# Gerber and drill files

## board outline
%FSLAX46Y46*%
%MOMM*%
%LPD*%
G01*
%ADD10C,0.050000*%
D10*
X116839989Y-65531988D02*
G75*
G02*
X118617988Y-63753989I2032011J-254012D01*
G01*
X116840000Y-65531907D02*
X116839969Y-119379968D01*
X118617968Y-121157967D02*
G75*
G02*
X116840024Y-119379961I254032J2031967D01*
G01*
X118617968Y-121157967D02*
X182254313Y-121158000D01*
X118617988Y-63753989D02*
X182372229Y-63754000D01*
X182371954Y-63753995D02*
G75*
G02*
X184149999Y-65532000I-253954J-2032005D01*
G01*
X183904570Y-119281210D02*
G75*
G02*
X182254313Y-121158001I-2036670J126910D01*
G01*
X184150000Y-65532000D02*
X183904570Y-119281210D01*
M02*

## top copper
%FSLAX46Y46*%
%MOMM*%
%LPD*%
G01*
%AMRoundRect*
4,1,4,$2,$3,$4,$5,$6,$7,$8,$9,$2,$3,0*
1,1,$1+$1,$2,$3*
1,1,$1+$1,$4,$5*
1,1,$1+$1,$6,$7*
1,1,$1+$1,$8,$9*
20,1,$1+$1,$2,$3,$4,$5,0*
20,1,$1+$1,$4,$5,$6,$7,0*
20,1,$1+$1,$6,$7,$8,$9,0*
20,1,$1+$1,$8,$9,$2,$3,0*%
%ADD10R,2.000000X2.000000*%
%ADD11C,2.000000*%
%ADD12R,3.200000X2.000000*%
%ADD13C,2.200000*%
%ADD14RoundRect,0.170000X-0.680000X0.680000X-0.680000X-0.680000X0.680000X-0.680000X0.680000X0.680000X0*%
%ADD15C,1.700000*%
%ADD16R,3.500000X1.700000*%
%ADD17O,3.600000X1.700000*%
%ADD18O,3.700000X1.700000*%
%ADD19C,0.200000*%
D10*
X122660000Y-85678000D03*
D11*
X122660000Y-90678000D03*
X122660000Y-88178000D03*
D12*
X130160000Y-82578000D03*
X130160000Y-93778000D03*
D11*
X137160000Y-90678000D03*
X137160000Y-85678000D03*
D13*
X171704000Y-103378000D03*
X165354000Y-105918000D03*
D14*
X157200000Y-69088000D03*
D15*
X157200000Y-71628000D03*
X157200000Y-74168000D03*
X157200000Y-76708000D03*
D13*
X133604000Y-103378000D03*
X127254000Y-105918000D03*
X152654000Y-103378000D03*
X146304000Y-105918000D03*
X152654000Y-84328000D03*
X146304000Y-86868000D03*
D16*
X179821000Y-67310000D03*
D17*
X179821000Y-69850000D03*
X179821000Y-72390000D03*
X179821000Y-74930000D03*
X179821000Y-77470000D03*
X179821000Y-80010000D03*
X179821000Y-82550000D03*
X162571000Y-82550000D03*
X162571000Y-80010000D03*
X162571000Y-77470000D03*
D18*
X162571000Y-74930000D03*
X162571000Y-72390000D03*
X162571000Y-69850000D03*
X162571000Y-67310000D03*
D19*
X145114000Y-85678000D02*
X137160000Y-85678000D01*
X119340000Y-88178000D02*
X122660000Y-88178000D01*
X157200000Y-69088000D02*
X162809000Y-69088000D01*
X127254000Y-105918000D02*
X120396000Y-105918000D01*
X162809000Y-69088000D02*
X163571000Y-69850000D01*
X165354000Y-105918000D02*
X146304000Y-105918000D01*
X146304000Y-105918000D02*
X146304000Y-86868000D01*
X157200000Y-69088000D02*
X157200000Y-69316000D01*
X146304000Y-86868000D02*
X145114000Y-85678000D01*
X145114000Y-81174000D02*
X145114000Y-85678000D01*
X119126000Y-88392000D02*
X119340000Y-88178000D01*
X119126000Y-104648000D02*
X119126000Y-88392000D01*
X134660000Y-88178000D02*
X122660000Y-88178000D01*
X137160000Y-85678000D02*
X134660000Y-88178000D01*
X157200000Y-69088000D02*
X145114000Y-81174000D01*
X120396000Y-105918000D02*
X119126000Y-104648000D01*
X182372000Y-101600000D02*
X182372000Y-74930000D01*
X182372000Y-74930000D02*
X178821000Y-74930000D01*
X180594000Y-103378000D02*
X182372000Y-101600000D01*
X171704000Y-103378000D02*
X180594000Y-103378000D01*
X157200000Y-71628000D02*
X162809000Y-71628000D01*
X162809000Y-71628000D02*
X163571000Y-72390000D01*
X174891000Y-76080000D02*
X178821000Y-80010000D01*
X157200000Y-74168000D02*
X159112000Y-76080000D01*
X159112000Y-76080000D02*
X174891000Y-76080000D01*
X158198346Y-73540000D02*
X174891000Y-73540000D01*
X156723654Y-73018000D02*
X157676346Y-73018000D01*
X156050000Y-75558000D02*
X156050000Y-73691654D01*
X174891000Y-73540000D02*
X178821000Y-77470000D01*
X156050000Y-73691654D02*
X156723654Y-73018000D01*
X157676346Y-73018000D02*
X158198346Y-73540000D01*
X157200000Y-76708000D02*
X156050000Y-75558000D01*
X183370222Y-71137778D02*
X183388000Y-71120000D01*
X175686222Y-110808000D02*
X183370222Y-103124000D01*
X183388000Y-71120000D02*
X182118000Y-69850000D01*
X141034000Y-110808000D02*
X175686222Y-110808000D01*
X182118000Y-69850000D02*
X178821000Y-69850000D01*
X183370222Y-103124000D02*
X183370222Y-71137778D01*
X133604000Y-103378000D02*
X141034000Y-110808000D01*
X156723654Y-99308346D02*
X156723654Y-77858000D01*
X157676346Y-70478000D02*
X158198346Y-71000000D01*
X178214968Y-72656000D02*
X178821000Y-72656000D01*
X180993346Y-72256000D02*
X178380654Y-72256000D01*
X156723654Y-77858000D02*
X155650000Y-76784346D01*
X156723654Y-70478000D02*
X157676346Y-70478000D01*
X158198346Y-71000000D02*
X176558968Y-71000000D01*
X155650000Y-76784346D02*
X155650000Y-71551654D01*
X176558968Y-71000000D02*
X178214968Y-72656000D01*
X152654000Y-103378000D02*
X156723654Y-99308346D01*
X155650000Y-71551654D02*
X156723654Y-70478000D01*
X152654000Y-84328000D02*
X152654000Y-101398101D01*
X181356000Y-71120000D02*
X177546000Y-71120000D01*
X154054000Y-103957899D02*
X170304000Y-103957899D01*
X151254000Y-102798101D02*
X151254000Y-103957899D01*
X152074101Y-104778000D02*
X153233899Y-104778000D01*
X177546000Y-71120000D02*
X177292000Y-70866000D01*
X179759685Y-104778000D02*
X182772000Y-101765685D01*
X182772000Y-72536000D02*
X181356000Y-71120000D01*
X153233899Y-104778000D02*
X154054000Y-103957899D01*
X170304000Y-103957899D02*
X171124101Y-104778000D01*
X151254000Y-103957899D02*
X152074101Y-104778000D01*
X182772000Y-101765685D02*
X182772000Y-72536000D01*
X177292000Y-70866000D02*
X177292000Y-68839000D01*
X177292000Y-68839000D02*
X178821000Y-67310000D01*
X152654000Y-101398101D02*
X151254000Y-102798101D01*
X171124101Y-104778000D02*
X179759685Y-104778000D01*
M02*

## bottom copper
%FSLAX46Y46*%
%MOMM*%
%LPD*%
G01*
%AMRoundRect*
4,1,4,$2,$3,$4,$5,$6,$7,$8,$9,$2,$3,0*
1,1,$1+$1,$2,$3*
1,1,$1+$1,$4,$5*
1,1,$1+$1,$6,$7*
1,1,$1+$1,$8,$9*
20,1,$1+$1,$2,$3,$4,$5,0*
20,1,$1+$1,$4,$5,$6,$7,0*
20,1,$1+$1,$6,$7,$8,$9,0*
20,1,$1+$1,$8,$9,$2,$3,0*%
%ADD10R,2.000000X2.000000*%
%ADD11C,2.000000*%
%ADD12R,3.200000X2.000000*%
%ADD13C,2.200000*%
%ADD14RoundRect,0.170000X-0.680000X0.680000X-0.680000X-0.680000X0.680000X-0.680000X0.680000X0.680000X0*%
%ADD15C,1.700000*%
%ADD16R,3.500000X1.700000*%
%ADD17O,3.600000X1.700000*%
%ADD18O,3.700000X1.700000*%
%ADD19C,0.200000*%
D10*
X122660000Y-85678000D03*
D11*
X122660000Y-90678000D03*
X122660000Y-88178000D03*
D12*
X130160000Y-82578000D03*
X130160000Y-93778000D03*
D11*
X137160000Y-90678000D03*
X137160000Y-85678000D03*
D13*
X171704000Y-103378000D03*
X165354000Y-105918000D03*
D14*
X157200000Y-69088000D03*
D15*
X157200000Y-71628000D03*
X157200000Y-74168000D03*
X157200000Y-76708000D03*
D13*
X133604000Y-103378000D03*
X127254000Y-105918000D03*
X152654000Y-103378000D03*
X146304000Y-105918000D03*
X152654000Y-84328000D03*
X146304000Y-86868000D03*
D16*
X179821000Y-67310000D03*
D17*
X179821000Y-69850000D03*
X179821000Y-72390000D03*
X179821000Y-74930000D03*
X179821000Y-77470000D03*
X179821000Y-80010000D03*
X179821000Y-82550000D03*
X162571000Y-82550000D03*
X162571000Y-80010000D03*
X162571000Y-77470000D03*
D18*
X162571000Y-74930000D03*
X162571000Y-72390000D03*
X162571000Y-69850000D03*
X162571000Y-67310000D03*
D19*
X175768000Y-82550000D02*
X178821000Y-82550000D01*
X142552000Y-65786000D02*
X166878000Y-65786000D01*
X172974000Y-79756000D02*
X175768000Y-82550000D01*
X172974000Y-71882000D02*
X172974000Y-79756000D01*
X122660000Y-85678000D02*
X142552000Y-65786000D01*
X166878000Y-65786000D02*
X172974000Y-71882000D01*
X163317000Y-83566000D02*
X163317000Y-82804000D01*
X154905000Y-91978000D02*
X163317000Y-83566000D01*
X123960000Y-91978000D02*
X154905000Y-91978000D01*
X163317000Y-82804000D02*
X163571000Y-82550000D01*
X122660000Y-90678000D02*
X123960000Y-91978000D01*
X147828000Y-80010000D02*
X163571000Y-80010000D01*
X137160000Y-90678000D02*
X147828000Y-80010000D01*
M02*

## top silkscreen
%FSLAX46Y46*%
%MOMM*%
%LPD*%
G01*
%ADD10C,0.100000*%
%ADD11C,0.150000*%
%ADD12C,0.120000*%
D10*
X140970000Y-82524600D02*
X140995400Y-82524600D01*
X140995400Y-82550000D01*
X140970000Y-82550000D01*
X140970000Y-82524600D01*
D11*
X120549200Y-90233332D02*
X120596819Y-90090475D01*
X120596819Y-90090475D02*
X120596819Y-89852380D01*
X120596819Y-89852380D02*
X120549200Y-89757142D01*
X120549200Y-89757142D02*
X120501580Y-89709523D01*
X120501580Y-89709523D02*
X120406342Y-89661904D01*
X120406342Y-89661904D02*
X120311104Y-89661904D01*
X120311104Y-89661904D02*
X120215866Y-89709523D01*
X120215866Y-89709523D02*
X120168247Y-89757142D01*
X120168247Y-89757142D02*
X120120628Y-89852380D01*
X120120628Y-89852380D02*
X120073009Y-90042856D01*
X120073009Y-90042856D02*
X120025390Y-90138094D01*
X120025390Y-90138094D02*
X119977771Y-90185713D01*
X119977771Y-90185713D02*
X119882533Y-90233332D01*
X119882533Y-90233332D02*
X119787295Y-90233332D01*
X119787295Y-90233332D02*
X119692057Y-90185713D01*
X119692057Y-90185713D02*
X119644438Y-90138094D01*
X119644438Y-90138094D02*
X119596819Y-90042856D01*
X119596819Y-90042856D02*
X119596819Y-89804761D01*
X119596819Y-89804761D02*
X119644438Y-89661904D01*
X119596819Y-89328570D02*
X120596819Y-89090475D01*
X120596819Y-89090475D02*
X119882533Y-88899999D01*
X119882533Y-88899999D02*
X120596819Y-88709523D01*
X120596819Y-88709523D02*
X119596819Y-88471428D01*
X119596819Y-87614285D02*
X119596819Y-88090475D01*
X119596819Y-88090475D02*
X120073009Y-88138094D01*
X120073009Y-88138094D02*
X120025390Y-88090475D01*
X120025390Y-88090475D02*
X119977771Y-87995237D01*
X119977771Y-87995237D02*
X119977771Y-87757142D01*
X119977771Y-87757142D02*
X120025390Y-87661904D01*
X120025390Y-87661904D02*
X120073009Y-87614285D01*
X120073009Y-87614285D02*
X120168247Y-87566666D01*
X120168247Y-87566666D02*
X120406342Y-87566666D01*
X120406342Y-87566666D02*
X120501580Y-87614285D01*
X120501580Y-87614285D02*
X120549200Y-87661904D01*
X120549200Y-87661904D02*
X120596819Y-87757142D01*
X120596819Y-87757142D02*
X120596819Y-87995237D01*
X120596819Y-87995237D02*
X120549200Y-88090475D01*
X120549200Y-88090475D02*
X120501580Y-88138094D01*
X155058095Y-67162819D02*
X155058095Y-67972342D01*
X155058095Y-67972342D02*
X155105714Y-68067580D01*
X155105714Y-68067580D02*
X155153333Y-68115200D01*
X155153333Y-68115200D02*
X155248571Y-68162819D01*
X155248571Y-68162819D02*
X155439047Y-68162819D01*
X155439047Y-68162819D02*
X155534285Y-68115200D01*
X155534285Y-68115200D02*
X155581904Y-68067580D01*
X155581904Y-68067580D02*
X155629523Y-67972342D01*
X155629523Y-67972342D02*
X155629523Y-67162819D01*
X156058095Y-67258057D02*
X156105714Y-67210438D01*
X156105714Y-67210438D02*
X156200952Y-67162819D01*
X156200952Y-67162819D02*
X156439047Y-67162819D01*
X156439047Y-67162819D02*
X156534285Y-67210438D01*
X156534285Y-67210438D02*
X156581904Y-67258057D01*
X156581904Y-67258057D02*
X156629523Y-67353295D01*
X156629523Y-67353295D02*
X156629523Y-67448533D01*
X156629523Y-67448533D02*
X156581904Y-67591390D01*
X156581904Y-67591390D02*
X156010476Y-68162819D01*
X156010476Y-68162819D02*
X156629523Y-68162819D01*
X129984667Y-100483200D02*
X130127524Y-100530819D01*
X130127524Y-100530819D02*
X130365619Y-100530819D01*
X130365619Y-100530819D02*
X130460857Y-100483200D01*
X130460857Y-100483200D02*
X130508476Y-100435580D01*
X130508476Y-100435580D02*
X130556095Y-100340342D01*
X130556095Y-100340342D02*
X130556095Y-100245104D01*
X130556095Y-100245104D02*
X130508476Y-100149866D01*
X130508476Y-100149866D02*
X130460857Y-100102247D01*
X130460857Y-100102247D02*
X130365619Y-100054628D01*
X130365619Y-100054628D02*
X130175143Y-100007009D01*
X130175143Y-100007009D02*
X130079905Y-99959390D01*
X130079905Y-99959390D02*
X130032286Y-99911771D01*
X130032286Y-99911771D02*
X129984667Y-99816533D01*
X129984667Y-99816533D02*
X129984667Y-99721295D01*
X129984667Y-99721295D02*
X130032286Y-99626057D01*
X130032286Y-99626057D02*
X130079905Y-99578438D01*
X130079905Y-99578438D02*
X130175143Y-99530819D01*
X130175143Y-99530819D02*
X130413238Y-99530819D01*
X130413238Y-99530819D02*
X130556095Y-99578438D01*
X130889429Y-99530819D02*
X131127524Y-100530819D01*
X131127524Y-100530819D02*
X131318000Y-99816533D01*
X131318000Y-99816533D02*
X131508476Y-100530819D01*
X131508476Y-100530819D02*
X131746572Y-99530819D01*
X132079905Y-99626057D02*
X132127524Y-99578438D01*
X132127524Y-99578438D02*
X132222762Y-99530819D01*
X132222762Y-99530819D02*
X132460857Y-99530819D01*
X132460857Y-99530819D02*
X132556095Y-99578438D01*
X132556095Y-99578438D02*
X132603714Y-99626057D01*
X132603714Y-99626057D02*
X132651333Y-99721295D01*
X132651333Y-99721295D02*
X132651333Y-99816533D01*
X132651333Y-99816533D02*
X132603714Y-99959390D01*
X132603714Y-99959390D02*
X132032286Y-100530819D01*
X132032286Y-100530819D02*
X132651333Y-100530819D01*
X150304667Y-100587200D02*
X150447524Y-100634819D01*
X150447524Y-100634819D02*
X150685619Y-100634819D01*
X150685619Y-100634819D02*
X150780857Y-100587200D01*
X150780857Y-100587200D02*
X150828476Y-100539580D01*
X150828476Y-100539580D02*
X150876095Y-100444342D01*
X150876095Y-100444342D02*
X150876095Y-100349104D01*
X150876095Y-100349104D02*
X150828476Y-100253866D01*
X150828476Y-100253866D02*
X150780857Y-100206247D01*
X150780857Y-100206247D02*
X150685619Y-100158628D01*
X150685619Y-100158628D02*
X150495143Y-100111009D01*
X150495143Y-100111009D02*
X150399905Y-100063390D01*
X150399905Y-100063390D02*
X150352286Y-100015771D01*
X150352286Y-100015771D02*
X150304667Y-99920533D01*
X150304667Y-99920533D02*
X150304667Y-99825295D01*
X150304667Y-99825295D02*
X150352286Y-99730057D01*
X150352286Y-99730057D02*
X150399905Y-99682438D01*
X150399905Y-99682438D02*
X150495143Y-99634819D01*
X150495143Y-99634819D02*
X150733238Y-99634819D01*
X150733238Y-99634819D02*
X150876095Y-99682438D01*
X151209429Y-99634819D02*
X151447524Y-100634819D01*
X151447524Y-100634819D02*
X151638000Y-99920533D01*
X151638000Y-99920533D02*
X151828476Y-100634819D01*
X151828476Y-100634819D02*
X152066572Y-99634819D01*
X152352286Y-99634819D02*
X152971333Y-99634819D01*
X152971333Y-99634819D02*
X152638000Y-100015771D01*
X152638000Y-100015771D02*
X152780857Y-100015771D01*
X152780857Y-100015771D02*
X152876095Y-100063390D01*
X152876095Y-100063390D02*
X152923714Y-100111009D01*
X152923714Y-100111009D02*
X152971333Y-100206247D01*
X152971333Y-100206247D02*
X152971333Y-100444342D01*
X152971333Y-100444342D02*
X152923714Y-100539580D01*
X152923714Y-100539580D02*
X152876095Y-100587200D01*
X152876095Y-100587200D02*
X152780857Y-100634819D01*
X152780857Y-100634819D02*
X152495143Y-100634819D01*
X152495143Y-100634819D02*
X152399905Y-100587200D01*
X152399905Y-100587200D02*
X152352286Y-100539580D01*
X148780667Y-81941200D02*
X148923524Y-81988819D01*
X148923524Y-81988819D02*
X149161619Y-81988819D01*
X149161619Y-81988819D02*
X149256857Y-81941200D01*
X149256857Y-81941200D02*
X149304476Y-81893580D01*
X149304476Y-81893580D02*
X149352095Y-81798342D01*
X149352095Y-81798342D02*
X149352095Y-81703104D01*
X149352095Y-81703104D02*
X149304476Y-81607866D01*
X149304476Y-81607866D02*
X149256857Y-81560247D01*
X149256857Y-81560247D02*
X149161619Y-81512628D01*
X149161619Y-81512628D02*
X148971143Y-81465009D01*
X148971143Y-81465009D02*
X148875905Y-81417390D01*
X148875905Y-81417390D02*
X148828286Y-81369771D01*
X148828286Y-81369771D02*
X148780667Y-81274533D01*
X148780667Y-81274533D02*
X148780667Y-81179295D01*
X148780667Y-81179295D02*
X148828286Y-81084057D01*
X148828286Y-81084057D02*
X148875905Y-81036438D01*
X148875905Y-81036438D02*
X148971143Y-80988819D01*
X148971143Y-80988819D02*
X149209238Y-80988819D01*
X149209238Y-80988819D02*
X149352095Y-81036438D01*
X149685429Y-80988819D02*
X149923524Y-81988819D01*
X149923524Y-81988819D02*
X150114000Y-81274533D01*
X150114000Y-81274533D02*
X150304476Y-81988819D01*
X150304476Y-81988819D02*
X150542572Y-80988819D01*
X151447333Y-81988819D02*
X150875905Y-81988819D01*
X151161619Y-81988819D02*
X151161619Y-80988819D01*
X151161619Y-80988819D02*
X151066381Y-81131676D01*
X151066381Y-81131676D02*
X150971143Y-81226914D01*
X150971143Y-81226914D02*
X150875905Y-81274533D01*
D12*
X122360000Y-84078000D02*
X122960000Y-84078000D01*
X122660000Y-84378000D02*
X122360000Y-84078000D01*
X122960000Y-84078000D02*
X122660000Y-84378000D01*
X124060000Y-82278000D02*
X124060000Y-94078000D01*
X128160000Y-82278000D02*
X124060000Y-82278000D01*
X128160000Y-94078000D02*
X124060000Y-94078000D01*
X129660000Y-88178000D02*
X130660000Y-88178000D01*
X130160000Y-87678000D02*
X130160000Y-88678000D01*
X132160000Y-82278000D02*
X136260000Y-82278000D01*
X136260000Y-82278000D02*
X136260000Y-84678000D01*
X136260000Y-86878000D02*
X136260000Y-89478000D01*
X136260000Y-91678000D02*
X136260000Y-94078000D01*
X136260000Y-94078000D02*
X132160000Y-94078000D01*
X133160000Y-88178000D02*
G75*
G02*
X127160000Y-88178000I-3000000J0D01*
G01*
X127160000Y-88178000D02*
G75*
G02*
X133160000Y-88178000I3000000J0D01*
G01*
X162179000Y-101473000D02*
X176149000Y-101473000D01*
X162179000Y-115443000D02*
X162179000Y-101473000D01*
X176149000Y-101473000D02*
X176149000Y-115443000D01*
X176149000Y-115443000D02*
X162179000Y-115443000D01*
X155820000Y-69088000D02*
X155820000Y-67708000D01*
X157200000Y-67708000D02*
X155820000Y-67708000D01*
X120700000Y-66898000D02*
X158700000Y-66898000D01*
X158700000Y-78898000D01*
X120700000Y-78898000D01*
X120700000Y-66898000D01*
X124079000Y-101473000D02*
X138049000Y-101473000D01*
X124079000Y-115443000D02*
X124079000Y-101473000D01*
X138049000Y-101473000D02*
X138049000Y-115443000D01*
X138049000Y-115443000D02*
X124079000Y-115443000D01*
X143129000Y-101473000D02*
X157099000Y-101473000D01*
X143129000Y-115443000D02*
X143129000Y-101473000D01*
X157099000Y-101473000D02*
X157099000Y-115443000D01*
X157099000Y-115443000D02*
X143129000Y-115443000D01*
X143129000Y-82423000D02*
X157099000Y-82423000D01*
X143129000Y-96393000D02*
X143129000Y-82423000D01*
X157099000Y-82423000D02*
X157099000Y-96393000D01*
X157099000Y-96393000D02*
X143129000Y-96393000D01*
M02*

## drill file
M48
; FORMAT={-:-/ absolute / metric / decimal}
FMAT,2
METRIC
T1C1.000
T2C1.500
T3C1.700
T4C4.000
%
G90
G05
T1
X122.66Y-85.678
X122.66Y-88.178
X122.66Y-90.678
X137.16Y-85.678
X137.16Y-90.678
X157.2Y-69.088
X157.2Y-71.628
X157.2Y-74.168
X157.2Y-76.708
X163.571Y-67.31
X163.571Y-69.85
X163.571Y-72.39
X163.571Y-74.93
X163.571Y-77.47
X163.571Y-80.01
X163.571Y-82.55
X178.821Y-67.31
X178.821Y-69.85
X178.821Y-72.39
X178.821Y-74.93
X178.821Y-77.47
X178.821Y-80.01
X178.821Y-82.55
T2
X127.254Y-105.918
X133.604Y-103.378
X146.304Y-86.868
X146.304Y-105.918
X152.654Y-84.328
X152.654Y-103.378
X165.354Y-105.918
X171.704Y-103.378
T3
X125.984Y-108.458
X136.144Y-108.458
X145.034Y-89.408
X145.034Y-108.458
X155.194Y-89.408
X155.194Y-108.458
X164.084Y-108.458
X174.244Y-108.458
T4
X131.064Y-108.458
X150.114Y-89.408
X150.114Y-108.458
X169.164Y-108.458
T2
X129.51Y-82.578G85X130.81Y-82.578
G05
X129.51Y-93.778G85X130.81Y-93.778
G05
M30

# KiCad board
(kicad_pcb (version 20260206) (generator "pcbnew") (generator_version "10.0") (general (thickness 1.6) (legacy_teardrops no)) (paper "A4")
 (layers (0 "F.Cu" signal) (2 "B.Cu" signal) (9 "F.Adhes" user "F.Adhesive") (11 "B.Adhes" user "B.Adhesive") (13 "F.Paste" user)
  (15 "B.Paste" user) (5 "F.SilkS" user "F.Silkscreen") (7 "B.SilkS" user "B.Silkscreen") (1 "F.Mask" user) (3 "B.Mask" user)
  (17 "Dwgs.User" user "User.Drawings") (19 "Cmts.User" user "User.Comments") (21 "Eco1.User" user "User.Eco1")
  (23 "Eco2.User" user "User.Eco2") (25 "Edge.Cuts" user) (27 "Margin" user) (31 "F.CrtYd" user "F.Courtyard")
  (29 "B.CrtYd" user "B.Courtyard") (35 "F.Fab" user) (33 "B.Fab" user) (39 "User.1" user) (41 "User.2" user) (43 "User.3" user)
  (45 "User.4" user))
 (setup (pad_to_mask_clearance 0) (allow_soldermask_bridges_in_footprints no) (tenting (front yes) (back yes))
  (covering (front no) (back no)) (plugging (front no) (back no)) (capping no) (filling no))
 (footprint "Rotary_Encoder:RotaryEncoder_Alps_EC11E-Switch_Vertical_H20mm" (layer "F.Cu") (at 122.66 85.678)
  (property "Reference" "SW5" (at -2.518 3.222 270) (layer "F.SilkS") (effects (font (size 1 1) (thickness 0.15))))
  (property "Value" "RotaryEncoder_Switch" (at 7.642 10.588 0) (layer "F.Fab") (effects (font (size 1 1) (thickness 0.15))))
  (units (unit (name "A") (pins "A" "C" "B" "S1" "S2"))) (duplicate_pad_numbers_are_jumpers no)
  (fp_line (start -0.3 -1.6) (end 0.3 -1.6) (stroke (width 0.12) (type solid)) (layer "F.SilkS"))
  (fp_line (start 0 -1.3) (end -0.3 -1.6) (stroke (width 0.12) (type solid)) (layer "F.SilkS"))
  (fp_line (start 0.3 -1.6) (end 0 -1.3) (stroke (width 0.12) (type solid)) (layer "F.SilkS"))
  (fp_line (start 1.4 -3.4) (end 1.4 8.4) (stroke (width 0.12) (type solid)) (layer "F.SilkS"))
  (fp_line (start 5.5 -3.4) (end 1.4 -3.4) (stroke (width 0.12) (type solid)) (layer "F.SilkS"))
  (fp_line (start 5.5 8.4) (end 1.4 8.4) (stroke (width 0.12) (type solid)) (layer "F.SilkS"))
  (fp_line (start 7 2.5) (end 8 2.5) (stroke (width 0.12) (type solid)) (layer "F.SilkS"))
  (fp_line (start 7.5 2) (end 7.5 3) (stroke (width 0.12) (type solid)) (layer "F.SilkS"))
  (fp_line (start 9.5 -3.4) (end 13.6 -3.4) (stroke (width 0.12) (type solid)) (layer "F.SilkS"))
  (fp_line (start 13.6 -3.4) (end 13.6 -1) (stroke (width 0.12) (type solid)) (layer "F.SilkS"))
  (fp_line (start 13.6 1.2) (end 13.6 3.8) (stroke (width 0.12) (type solid)) (layer "F.SilkS"))
  (fp_line (start 13.6 6) (end 13.6 8.4) (stroke (width 0.12) (type solid)) (layer "F.SilkS"))
  (fp_line (start 13.6 8.4) (end 9.5 8.4) (stroke (width 0.12) (type solid)) (layer "F.SilkS"))
  (fp_circle (center 7.5 2.5) (end 10.5 2.5) (stroke (width 0.12) (type solid)) (fill no) (layer "F.SilkS"))
  (pad "A" thru_hole rect (at 0 0) (size 2 2) (drill 1) (layers "*.Cu" "*.Mask") (remove_unused_layers no) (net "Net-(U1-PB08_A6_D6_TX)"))
  (pad "B" thru_hole circle (at 0 5) (size 2 2) (drill 1) (layers "*.Cu" "*.Mask") (remove_unused_layers no) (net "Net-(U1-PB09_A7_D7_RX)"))
  (pad "C" thru_hole circle (at 0 2.5) (size 2 2) (drill 1) (layers "*.Cu" "*.Mask") (remove_unused_layers no) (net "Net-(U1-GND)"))
  (pad "MP" thru_hole rect (at 7.5 -3.1) (size 3.2 2) (drill oval 2.8 1.5) (layers "*.Cu" "*.Mask") (remove_unused_layers no))
  (pad "MP" thru_hole rect (at 7.5 8.1) (size 3.2 2) (drill oval 2.8 1.5) (layers "*.Cu" "*.Mask") (remove_unused_layers no))
  (pad "S1" thru_hole circle (at 14.5 5) (size 2 2) (drill 1) (layers "*.Cu" "*.Mask") (remove_unused_layers no)
   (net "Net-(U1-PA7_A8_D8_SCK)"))
  (pad "S2" thru_hole circle (at 14.5 0) (size 2 2) (drill 1) (layers "*.Cu" "*.Mask") (remove_unused_layers no) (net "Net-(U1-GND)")))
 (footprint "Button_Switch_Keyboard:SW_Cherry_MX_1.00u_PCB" (layer "F.Cu") (at 171.704 103.378)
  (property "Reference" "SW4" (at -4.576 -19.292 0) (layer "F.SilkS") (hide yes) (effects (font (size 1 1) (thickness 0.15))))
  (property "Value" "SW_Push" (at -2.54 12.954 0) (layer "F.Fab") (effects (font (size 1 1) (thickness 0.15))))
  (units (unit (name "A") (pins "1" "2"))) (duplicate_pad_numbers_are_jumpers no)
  (fp_line (start -9.525 -1.905) (end 4.445 -1.905) (stroke (width 0.12) (type solid)) (layer "F.SilkS"))
  (fp_line (start -9.525 12.065) (end -9.525 -1.905) (stroke (width 0.12) (type solid)) (layer "F.SilkS"))
  (fp_line (start 4.445 -1.905) (end 4.445 12.065) (stroke (width 0.12) (type solid)) (layer "F.SilkS"))
  (fp_line (start 4.445 12.065) (end -9.525 12.065) (stroke (width 0.12) (type solid)) (layer "F.SilkS"))
  (pad "" np_thru_hole circle (at -7.62 5.08) (size 1.7 1.7) (drill 1.7) (layers "*.Cu" "*.Mask"))
  (pad "" np_thru_hole circle (at -2.54 5.08) (size 4 4) (drill 4) (layers "*.Cu" "*.Mask"))
  (pad "" np_thru_hole circle (at 2.54 5.08) (size 1.7 1.7) (drill 1.7) (layers "*.Cu" "*.Mask"))
  (pad "1" thru_hole circle (at 0 0) (size 2.2 2.2) (drill 1.5) (layers "*.Cu" "*.Mask") (remove_unused_layers no)
   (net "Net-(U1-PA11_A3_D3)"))
  (pad "2" thru_hole circle (at -6.35 2.54) (size 2.2 2.2) (drill 1.5) (layers "*.Cu" "*.Mask") (remove_unused_layers no)
   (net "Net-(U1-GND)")))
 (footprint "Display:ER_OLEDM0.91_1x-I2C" (layer "F.Cu") (at 157.2 69.088 -90)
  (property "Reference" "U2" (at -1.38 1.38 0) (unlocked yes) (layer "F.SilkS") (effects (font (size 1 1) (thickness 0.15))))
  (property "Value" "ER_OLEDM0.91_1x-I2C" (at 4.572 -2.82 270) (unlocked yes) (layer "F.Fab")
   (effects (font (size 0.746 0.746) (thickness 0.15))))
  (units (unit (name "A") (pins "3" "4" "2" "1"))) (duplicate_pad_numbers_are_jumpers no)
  (fp_line (start 0 1.38) (end -1.38 1.38) (stroke (width 0.12) (type solid)) (layer "F.SilkS"))
  (fp_line (start -1.38 0) (end -1.38 1.38) (stroke (width 0.12) (type solid)) (layer "F.SilkS"))
  (fp_rect (start -2.19 -1.5) (end 9.81 36.5) (stroke (width 0.12) (type solid)) (fill no) (layer "F.SilkS"))
  (pad "1" thru_hole roundrect (at 0 0 270) (size 1.7 1.7) (drill 1) (layers "*.Cu" "*.Mask") (remove_unused_layers no)
   (roundrect_rratio 0.1) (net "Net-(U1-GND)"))
  (pad "2" thru_hole circle (at 2.54 0 270) (size 1.7 1.7) (drill 1) (layers "*.Cu" "*.Mask") (remove_unused_layers no) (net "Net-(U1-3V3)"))
  (pad "3" thru_hole circle (at 5.08 0 270) (size 1.7 1.7) (drill 1) (layers "*.Cu" "*.Mask") (remove_unused_layers no)
   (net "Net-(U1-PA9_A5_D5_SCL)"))
  (pad "4" thru_hole circle (at 7.62 0 270) (size 1.7 1.7) (drill 1) (layers "*.Cu" "*.Mask") (remove_unused_layers no)
   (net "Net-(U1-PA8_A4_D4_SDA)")))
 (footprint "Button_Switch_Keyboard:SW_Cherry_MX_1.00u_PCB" (layer "F.Cu") (at 133.604 103.378)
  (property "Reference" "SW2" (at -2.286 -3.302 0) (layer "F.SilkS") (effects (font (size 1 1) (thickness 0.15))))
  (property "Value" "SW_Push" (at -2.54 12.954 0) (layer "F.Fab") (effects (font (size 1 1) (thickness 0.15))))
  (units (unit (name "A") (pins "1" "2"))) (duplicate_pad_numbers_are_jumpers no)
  (fp_line (start -9.525 -1.905) (end 4.445 -1.905) (stroke (width 0.12) (type solid)) (layer "F.SilkS"))
  (fp_line (start -9.525 12.065) (end -9.525 -1.905) (stroke (width 0.12) (type solid)) (layer "F.SilkS"))
  (fp_line (start 4.445 -1.905) (end 4.445 12.065) (stroke (width 0.12) (type solid)) (layer "F.SilkS"))
  (fp_line (start 4.445 12.065) (end -9.525 12.065) (stroke (width 0.12) (type solid)) (layer "F.SilkS"))
  (pad "" np_thru_hole circle (at -7.62 5.08) (size 1.7 1.7) (drill 1.7) (layers "*.Cu" "*.Mask"))
  (pad "" np_thru_hole circle (at -2.54 5.08) (size 4 4) (drill 4) (layers "*.Cu" "*.Mask"))
  (pad "" np_thru_hole circle (at 2.54 5.08) (size 1.7 1.7) (drill 1.7) (layers "*.Cu" "*.Mask"))
  (pad "1" thru_hole circle (at 0 0) (size 2.2 2.2) (drill 1.5) (layers "*.Cu" "*.Mask") (remove_unused_layers no)
   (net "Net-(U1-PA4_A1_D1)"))
  (pad "2" thru_hole circle (at -6.35 2.54) (size 2.2 2.2) (drill 1.5) (layers "*.Cu" "*.Mask") (remove_unused_layers no)
   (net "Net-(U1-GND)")))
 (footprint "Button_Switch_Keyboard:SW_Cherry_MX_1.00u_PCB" (layer "F.Cu") (at 152.654 103.378)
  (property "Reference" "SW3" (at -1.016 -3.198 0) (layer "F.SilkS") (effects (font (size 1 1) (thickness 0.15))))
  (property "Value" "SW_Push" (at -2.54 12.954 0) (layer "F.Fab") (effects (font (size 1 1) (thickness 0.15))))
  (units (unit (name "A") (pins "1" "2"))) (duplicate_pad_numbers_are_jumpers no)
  (fp_line (start -9.525 -1.905) (end 4.445 -1.905) (stroke (width 0.12) (type solid)) (layer "F.SilkS"))
  (fp_line (start -9.525 12.065) (end -9.525 -1.905) (stroke (width 0.12) (type solid)) (layer "F.SilkS"))
  (fp_line (start 4.445 -1.905) (end 4.445 12.065) (stroke (width 0.12) (type solid)) (layer "F.SilkS"))
  (fp_line (start 4.445 12.065) (end -9.525 12.065) (stroke (width 0.12) (type solid)) (layer "F.SilkS"))
  (pad "" np_thru_hole circle (at -7.62 5.08) (size 1.7 1.7) (drill 1.7) (layers "*.Cu" "*.Mask"))
  (pad "" np_thru_hole circle (at -2.54 5.08) (size 4 4) (drill 4) (layers "*.Cu" "*.Mask"))
  (pad "" np_thru_hole circle (at 2.54 5.08) (size 1.7 1.7) (drill 1.7) (layers "*.Cu" "*.Mask"))
  (pad "1" thru_hole circle (at 0 0) (size 2.2 2.2) (drill 1.5) (layers "*.Cu" "*.Mask") (remove_unused_layers no)
   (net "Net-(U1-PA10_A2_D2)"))
  (pad "2" thru_hole circle (at -6.35 2.54) (size 2.2 2.2) (drill 1.5) (layers "*.Cu" "*.Mask") (remove_unused_layers no)
   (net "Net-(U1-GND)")))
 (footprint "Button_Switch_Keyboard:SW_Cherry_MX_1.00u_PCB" (layer "F.Cu") (at 152.654 84.328)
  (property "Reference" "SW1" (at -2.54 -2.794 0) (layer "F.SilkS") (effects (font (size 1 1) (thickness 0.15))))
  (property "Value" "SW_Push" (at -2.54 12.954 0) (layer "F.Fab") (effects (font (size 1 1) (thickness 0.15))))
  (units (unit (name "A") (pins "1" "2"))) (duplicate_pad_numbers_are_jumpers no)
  (fp_line (start -9.525 -1.905) (end 4.445 -1.905) (stroke (width 0.12) (type solid)) (layer "F.SilkS"))
  (fp_line (start -9.525 12.065) (end -9.525 -1.905) (stroke (width 0.12) (type solid)) (layer "F.SilkS"))
  (fp_line (start 4.445 -1.905) (end 4.445 12.065) (stroke (width 0.12) (type solid)) (layer "F.SilkS"))
  (fp_line (start 4.445 12.065) (end -9.525 12.065) (stroke (width 0.12) (type solid)) (layer "F.SilkS"))
  (pad "" np_thru_hole circle (at -7.62 5.08) (size 1.7 1.7) (drill 1.7) (layers "*.Cu" "*.Mask"))
  (pad "" np_thru_hole circle (at -2.54 5.08) (size 4 4) (drill 4) (layers "*.Cu" "*.Mask"))
  (pad "" np_thru_hole circle (at 2.54 5.08) (size 1.7 1.7) (drill 1.7) (layers "*.Cu" "*.Mask"))
  (pad "1" thru_hole circle (at 0 0) (size 2.2 2.2) (drill 1.5) (layers "*.Cu" "*.Mask") (remove_unused_layers no)
   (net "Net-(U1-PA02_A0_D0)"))
  (pad "2" thru_hole circle (at -6.35 2.54) (size 2.2 2.2) (drill 1.5) (layers "*.Cu" "*.Mask") (remove_unused_layers no)
   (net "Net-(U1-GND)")))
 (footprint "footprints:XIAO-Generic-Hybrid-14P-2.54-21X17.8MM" (layer "B.Cu") (at 171.196 74.93 180)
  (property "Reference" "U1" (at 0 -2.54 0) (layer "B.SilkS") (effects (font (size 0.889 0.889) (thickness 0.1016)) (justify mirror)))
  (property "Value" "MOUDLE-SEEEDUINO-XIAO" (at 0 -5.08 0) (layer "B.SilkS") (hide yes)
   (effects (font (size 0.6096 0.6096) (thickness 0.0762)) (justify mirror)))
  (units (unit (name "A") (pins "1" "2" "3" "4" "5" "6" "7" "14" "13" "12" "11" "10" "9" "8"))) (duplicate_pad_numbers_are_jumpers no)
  (pad "1" thru_hole rect (at -7.625 7.62 180) (size 3.5 1.7) (drill 1 (offset -1 0)) (layers "*.Cu" "*.Mask") (remove_unused_layers no)
   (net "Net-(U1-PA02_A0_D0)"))
  (pad "2" thru_hole oval (at -7.625 5.08 180) (size 3.6 1.7) (drill 1 (offset -1 0)) (layers "*.Cu" "*.Mask") (remove_unused_layers no)
   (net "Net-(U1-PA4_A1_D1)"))
  (pad "3" thru_hole oval (at -7.625 2.54 180) (size 3.6 1.7) (drill 1 (offset -1 0)) (layers "*.Cu" "*.Mask") (remove_unused_layers no)
   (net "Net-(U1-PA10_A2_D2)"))
  (pad "4" thru_hole oval (at -7.625 0 180) (size 3.6 1.7) (drill 1 (offset -1 0)) (layers "*.Cu" "*.Mask") (remove_unused_layers no)
   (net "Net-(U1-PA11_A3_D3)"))
  (pad "5" thru_hole oval (at -7.625 -2.54 180) (size 3.6 1.7) (drill 1 (offset -1 0)) (layers "*.Cu" "*.Mask") (remove_unused_layers no)
   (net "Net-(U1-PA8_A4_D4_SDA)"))
  (pad "6" thru_hole oval (at -7.625 -5.08) (size 3.6 1.7) (drill 1 (offset 1 0)) (layers "*.Cu" "*.Mask") (remove_unused_layers no)
   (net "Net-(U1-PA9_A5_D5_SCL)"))
  (pad "7" thru_hole oval (at -7.625 -7.62 180) (size 3.6 1.7) (drill 1 (offset -1 0)) (layers "*.Cu" "*.Mask") (remove_unused_layers no)
   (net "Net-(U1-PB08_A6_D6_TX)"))
  (pad "8" thru_hole oval (at 7.625 -7.62 180) (size 3.6 1.7) (drill 1 (offset 1 0)) (layers "*.Cu" "*.Mask") (remove_unused_layers no)
   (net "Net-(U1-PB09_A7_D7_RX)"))
  (pad "9" thru_hole oval (at 7.625 -5.08 180) (size 3.6 1.7) (drill 1 (offset 1 0)) (layers "*.Cu" "*.Mask") (remove_unused_layers no)
   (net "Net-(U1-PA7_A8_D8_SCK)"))
  (pad "10" thru_hole oval (at 7.625 -2.54 180) (size 3.6 1.7) (drill 1 (offset 1 0)) (layers "*.Cu" "*.Mask") (remove_unused_layers no)
   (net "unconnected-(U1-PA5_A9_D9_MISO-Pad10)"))
  (pad "11" thru_hole oval (at 7.625 0 180) (size 3.7 1.7) (drill 1 (offset 1 0)) (layers "*.Cu" "*.Mask") (remove_unused_layers no)
   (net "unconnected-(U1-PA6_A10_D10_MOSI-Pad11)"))
  (pad "12" thru_hole oval (at 7.625 2.54 180) (size 3.7 1.7) (drill 1 (offset 1 0)) (layers "*.Cu" "*.Mask") (remove_unused_layers no)
   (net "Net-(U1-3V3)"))
  (pad "13" thru_hole oval (at 7.625 5.08 180) (size 3.7 1.7) (drill 1 (offset 1 0)) (layers "*.Cu" "*.Mask") (remove_unused_layers no)
   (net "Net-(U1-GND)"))
  (pad "14" thru_hole oval (at 7.625 7.62 180) (size 3.7 1.7) (drill 1 (offset 1 0)) (layers "*.Cu" "*.Mask") (remove_unused_layers no)
   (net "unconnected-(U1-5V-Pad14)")))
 (gr_rect (start 140.97 82.5246) (end 140.9954 82.55) (stroke (width 0.1) (type default)) (fill no) (layer "F.SilkS"))
 (gr_arc (start 116.839989 65.531988) (mid 117.423966 64.337966) (end 118.617988 63.753989) (stroke (width 0.05) (type default))
  (layer "Edge.Cuts"))
 (gr_line (start 116.84 65.531907) (end 116.839969 119.379968) (stroke (width 0.05) (type default)) (layer "Edge.Cuts"))
 (gr_arc (start 118.617968 121.157967) (mid 117.423946 120.57399) (end 116.839969 119.379968) (stroke (width 0.05) (type default))
  (layer "Edge.Cuts"))
 (gr_line (start 118.617968 121.157967) (end 182.254313 121.158) (stroke (width 0.05) (type default)) (layer "Edge.Cuts"))
 (gr_line (start 118.617988 63.753989) (end 182.372229 63.754) (stroke (width 0.05) (type default)) (layer "Edge.Cuts"))
 (gr_arc (start 182.371954 63.753995) (mid 183.566006 64.337961) (end 184.15 65.532) (stroke (width 0.05) (type default))
  (layer "Edge.Cuts"))
 (gr_arc (start 183.90457 119.28121) (mid 183.400355 120.501784) (end 182.254313 121.158) (stroke (width 0.05) (type default))
  (layer "Edge.Cuts"))
 (gr_line (start 184.15 65.532) (end 183.90457 119.28121) (stroke (width 0.05) (type default)) (layer "Edge.Cuts"))
 (segment (start 175.768 82.55) (end 178.821 82.55) (width 0.2) (layer "B.Cu") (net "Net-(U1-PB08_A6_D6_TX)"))
 (segment (start 142.552 65.786) (end 166.878 65.786) (width 0.2) (layer "B.Cu") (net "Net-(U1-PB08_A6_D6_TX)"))
 (segment (start 172.974 79.756) (end 175.768 82.55) (width 0.2) (layer "B.Cu") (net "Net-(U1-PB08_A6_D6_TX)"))
 (segment (start 172.974 71.882) (end 172.974 79.756) (width 0.2) (layer "B.Cu") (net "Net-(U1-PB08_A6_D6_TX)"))
 (segment (start 122.66 85.678) (end 142.552 65.786) (width 0.2) (layer "B.Cu") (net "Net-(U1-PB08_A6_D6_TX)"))
 (segment (start 166.878 65.786) (end 172.974 71.882) (width 0.2) (layer "B.Cu") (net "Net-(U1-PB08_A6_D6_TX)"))
 (segment (start 163.317 83.566) (end 163.317 82.804) (width 0.2) (layer "B.Cu") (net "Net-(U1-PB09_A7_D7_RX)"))
 (segment (start 154.905 91.978) (end 163.317 83.566) (width 0.2) (layer "B.Cu") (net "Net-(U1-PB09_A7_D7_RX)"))
 (segment (start 123.96 91.978) (end 154.905 91.978) (width 0.2) (layer "B.Cu") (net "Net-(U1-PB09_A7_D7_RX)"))
 (segment (start 163.317 82.804) (end 163.571 82.55) (width 0.2) (layer "B.Cu") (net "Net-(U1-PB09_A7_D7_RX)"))
 (segment (start 122.66 90.678) (end 123.96 91.978) (width 0.2) (layer "B.Cu") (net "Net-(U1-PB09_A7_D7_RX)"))
 (segment (start 145.114 85.678) (end 137.16 85.678) (width 0.2) (layer "F.Cu") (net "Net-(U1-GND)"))
 (segment (start 119.34 88.178) (end 122.66 88.178) (width 0.2) (layer "F.Cu") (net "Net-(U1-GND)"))
 (segment (start 157.2 69.088) (end 162.809 69.088) (width 0.2) (layer "F.Cu") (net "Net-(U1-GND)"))
 (segment (start 127.254 105.918) (end 120.396 105.918) (width 0.2) (layer "F.Cu") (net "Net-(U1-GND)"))
 (segment (start 162.809 69.088) (end 163.571 69.85) (width 0.2) (layer "F.Cu") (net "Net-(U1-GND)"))
 (segment (start 165.354 105.918) (end 146.304 105.918) (width 0.2) (layer "F.Cu") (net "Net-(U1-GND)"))
 (segment (start 146.304 105.918) (end 146.304 86.868) (width 0.2) (layer "F.Cu") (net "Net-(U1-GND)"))
 (segment (start 157.2 69.088) (end 157.2 69.316) (width 0.2) (layer "F.Cu") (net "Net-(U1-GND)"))
 (segment (start 146.304 86.868) (end 145.114 85.678) (width 0.2) (layer "F.Cu") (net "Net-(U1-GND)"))
 (segment (start 145.114 81.174) (end 145.114 85.678) (width 0.2) (layer "F.Cu") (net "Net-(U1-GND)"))
 (segment (start 119.126 88.392) (end 119.34 88.178) (width 0.2) (layer "F.Cu") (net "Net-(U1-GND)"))
 (segment (start 119.126 104.648) (end 119.126 88.392) (width 0.2) (layer "F.Cu") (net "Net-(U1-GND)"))
 (segment (start 134.66 88.178) (end 122.66 88.178) (width 0.2) (layer "F.Cu") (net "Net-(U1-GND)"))
 (segment (start 137.16 85.678) (end 134.66 88.178) (width 0.2) (layer "F.Cu") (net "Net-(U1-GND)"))
 (segment (start 157.2 69.088) (end 145.114 81.174) (width 0.2) (layer "F.Cu") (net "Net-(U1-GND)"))
 (segment (start 120.396 105.918) (end 119.126 104.648) (width 0.2) (layer "F.Cu") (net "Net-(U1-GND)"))
 (segment (start 147.828 80.01) (end 163.571 80.01) (width 0.2) (layer "B.Cu") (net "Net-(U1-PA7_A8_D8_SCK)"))
 (segment (start 137.16 90.678) (end 147.828 80.01) (width 0.2) (layer "B.Cu") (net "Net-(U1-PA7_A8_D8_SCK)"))
 (segment (start 182.372 101.6) (end 182.372 74.93) (width 0.2) (layer "F.Cu") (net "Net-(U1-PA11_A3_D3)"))
 (segment (start 182.372 74.93) (end 178.821 74.93) (width 0.2) (layer "F.Cu") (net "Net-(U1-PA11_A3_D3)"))
 (segment (start 180.594 103.378) (end 182.372 101.6) (width 0.2) (layer "F.Cu") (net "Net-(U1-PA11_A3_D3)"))
 (segment (start 171.704 103.378) (end 180.594 103.378) (width 0.2) (layer "F.Cu") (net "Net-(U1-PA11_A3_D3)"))
 (segment (start 157.2 71.628) (end 162.809 71.628) (width 0.2) (layer "F.Cu") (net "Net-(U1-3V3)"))
 (segment (start 162.809 71.628) (end 163.571 72.39) (width 0.2) (layer "F.Cu") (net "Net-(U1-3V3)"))
 (segment (start 174.891 76.08) (end 178.821 80.01) (width 0.2) (layer "F.Cu") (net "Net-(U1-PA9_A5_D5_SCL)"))
 (segment (start 157.2 74.168) (end 159.112 76.08) (width 0.2) (layer "F.Cu") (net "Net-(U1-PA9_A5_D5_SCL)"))
 (segment (start 159.112 76.08) (end 174.891 76.08) (width 0.2) (layer "F.Cu") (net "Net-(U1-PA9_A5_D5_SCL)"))
 (segment (start 158.198346 73.54) (end 174.891 73.54) (width 0.2) (layer "F.Cu") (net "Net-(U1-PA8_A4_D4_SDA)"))
 (segment (start 156.723654 73.018) (end 157.676346 73.018) (width 0.2) (layer "F.Cu") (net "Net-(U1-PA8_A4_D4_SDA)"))
 (segment (start 156.05 75.558) (end 156.05 73.691654) (width 0.2) (layer "F.Cu") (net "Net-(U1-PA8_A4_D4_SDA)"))
 (segment (start 174.891 73.54) (end 178.821 77.47) (width 0.2) (layer "F.Cu") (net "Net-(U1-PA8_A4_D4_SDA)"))
 (segment (start 156.05 73.691654) (end 156.723654 73.018) (width 0.2) (layer "F.Cu") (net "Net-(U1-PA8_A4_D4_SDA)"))
 (segment (start 157.676346 73.018) (end 158.198346 73.54) (width 0.2) (layer "F.Cu") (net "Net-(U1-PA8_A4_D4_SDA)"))
 (segment (start 157.2 76.708) (end 156.05 75.558) (width 0.2) (layer "F.Cu") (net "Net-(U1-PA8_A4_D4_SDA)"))
 (segment (start 183.370222 71.137778) (end 183.388 71.12) (width 0.2) (layer "F.Cu") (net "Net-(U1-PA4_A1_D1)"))
 (segment (start 175.686222 110.808) (end 183.370222 103.124) (width 0.2) (layer "F.Cu") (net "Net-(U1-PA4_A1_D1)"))
 (segment (start 183.388 71.12) (end 182.118 69.85) (width 0.2) (layer "F.Cu") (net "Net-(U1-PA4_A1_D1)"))
 (segment (start 141.034 110.808) (end 175.686222 110.808) (width 0.2) (layer "F.Cu") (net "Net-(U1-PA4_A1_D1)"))
 (segment (start 182.118 69.85) (end 178.821 69.85) (width 0.2) (layer "F.Cu") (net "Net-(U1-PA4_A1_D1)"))
 (segment (start 183.370222 103.124) (end 183.370222 71.137778) (width 0.2) (layer "F.Cu") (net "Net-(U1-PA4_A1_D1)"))
 (segment (start 133.604 103.378) (end 141.034 110.808) (width 0.2) (layer "F.Cu") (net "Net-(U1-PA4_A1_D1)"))
 (segment (start 156.723654 99.308346) (end 156.723654 77.858) (width 0.2) (layer "F.Cu") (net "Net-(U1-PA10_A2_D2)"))
 (segment (start 157.676346 70.478) (end 158.198346 71) (width 0.2) (layer "F.Cu") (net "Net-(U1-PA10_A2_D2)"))
 (segment (start 178.214968 72.656) (end 178.821 72.656) (width 0.2) (layer "F.Cu") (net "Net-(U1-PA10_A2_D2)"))
 (segment (start 180.993346 72.256) (end 178.380654 72.256) (width 0.2) (layer "F.Cu") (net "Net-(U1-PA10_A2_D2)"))
 (segment (start 156.723654 77.858) (end 155.65 76.784346) (width 0.2) (layer "F.Cu") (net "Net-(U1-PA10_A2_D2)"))
 (segment (start 156.723654 70.478) (end 157.676346 70.478) (width 0.2) (layer "F.Cu") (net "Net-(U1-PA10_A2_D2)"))
 (segment (start 158.198346 71) (end 176.558968 71) (width 0.2) (layer "F.Cu") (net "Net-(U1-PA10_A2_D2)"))
 (segment (start 155.65 76.784346) (end 155.65 71.551654) (width 0.2) (layer "F.Cu") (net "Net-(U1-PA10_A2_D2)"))
 (segment (start 176.558968 71) (end 178.214968 72.656) (width 0.2) (layer "F.Cu") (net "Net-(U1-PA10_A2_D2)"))
 (segment (start 152.654 103.378) (end 156.723654 99.308346) (width 0.2) (layer "F.Cu") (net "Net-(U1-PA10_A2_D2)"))
 (segment (start 155.65 71.551654) (end 156.723654 70.478) (width 0.2) (layer "F.Cu") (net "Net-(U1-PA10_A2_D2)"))
 (segment (start 152.654 84.328) (end 152.654 101.398101) (width 0.2) (layer "F.Cu") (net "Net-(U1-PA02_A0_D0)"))
 (segment (start 181.356 71.12) (end 177.546 71.12) (width 0.2) (layer "F.Cu") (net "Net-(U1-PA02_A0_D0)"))
 (segment (start 154.054 103.957899) (end 170.304 103.957899) (width 0.2) (layer "F.Cu") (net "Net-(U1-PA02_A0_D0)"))
 (segment (start 151.254 102.798101) (end 151.254 103.957899) (width 0.2) (layer "F.Cu") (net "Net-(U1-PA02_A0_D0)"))
 (segment (start 152.074101 104.778) (end 153.233899 104.778) (width 0.2) (layer "F.Cu") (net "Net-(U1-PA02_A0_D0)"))
 (segment (start 177.546 71.12) (end 177.292 70.866) (width 0.2) (layer "F.Cu") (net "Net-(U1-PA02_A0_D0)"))
 (segment (start 179.759685 104.778) (end 182.772 101.765685) (width 0.2) (layer "F.Cu") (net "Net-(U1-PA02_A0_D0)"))
 (segment (start 182.772 72.536) (end 181.356 71.12) (width 0.2) (layer "F.Cu") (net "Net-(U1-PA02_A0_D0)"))
 (segment (start 153.233899 104.778) (end 154.054 103.957899) (width 0.2) (layer "F.Cu") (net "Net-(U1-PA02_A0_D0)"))
 (segment (start 170.304 103.957899) (end 171.124101 104.778) (width 0.2) (layer "F.Cu") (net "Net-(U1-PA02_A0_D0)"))
 (segment (start 151.254 103.957899) (end 152.074101 104.778) (width 0.2) (layer "F.Cu") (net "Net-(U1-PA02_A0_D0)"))
 (segment (start 182.772 101.765685) (end 182.772 72.536) (width 0.2) (layer "F.Cu") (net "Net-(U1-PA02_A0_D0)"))
 (segment (start 177.292 70.866) (end 177.292 68.839) (width 0.2) (layer "F.Cu") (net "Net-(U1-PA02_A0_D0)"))
 (segment (start 177.292 68.839) (end 178.821 67.31) (width 0.2) (layer "F.Cu") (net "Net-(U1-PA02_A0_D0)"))
 (segment (start 152.654 101.398101) (end 151.254 102.798101) (width 0.2) (layer "F.Cu") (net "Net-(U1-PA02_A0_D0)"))
 (segment (start 171.124101 104.778) (end 179.759685 104.778) (width 0.2) (layer "F.Cu") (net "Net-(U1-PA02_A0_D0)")))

